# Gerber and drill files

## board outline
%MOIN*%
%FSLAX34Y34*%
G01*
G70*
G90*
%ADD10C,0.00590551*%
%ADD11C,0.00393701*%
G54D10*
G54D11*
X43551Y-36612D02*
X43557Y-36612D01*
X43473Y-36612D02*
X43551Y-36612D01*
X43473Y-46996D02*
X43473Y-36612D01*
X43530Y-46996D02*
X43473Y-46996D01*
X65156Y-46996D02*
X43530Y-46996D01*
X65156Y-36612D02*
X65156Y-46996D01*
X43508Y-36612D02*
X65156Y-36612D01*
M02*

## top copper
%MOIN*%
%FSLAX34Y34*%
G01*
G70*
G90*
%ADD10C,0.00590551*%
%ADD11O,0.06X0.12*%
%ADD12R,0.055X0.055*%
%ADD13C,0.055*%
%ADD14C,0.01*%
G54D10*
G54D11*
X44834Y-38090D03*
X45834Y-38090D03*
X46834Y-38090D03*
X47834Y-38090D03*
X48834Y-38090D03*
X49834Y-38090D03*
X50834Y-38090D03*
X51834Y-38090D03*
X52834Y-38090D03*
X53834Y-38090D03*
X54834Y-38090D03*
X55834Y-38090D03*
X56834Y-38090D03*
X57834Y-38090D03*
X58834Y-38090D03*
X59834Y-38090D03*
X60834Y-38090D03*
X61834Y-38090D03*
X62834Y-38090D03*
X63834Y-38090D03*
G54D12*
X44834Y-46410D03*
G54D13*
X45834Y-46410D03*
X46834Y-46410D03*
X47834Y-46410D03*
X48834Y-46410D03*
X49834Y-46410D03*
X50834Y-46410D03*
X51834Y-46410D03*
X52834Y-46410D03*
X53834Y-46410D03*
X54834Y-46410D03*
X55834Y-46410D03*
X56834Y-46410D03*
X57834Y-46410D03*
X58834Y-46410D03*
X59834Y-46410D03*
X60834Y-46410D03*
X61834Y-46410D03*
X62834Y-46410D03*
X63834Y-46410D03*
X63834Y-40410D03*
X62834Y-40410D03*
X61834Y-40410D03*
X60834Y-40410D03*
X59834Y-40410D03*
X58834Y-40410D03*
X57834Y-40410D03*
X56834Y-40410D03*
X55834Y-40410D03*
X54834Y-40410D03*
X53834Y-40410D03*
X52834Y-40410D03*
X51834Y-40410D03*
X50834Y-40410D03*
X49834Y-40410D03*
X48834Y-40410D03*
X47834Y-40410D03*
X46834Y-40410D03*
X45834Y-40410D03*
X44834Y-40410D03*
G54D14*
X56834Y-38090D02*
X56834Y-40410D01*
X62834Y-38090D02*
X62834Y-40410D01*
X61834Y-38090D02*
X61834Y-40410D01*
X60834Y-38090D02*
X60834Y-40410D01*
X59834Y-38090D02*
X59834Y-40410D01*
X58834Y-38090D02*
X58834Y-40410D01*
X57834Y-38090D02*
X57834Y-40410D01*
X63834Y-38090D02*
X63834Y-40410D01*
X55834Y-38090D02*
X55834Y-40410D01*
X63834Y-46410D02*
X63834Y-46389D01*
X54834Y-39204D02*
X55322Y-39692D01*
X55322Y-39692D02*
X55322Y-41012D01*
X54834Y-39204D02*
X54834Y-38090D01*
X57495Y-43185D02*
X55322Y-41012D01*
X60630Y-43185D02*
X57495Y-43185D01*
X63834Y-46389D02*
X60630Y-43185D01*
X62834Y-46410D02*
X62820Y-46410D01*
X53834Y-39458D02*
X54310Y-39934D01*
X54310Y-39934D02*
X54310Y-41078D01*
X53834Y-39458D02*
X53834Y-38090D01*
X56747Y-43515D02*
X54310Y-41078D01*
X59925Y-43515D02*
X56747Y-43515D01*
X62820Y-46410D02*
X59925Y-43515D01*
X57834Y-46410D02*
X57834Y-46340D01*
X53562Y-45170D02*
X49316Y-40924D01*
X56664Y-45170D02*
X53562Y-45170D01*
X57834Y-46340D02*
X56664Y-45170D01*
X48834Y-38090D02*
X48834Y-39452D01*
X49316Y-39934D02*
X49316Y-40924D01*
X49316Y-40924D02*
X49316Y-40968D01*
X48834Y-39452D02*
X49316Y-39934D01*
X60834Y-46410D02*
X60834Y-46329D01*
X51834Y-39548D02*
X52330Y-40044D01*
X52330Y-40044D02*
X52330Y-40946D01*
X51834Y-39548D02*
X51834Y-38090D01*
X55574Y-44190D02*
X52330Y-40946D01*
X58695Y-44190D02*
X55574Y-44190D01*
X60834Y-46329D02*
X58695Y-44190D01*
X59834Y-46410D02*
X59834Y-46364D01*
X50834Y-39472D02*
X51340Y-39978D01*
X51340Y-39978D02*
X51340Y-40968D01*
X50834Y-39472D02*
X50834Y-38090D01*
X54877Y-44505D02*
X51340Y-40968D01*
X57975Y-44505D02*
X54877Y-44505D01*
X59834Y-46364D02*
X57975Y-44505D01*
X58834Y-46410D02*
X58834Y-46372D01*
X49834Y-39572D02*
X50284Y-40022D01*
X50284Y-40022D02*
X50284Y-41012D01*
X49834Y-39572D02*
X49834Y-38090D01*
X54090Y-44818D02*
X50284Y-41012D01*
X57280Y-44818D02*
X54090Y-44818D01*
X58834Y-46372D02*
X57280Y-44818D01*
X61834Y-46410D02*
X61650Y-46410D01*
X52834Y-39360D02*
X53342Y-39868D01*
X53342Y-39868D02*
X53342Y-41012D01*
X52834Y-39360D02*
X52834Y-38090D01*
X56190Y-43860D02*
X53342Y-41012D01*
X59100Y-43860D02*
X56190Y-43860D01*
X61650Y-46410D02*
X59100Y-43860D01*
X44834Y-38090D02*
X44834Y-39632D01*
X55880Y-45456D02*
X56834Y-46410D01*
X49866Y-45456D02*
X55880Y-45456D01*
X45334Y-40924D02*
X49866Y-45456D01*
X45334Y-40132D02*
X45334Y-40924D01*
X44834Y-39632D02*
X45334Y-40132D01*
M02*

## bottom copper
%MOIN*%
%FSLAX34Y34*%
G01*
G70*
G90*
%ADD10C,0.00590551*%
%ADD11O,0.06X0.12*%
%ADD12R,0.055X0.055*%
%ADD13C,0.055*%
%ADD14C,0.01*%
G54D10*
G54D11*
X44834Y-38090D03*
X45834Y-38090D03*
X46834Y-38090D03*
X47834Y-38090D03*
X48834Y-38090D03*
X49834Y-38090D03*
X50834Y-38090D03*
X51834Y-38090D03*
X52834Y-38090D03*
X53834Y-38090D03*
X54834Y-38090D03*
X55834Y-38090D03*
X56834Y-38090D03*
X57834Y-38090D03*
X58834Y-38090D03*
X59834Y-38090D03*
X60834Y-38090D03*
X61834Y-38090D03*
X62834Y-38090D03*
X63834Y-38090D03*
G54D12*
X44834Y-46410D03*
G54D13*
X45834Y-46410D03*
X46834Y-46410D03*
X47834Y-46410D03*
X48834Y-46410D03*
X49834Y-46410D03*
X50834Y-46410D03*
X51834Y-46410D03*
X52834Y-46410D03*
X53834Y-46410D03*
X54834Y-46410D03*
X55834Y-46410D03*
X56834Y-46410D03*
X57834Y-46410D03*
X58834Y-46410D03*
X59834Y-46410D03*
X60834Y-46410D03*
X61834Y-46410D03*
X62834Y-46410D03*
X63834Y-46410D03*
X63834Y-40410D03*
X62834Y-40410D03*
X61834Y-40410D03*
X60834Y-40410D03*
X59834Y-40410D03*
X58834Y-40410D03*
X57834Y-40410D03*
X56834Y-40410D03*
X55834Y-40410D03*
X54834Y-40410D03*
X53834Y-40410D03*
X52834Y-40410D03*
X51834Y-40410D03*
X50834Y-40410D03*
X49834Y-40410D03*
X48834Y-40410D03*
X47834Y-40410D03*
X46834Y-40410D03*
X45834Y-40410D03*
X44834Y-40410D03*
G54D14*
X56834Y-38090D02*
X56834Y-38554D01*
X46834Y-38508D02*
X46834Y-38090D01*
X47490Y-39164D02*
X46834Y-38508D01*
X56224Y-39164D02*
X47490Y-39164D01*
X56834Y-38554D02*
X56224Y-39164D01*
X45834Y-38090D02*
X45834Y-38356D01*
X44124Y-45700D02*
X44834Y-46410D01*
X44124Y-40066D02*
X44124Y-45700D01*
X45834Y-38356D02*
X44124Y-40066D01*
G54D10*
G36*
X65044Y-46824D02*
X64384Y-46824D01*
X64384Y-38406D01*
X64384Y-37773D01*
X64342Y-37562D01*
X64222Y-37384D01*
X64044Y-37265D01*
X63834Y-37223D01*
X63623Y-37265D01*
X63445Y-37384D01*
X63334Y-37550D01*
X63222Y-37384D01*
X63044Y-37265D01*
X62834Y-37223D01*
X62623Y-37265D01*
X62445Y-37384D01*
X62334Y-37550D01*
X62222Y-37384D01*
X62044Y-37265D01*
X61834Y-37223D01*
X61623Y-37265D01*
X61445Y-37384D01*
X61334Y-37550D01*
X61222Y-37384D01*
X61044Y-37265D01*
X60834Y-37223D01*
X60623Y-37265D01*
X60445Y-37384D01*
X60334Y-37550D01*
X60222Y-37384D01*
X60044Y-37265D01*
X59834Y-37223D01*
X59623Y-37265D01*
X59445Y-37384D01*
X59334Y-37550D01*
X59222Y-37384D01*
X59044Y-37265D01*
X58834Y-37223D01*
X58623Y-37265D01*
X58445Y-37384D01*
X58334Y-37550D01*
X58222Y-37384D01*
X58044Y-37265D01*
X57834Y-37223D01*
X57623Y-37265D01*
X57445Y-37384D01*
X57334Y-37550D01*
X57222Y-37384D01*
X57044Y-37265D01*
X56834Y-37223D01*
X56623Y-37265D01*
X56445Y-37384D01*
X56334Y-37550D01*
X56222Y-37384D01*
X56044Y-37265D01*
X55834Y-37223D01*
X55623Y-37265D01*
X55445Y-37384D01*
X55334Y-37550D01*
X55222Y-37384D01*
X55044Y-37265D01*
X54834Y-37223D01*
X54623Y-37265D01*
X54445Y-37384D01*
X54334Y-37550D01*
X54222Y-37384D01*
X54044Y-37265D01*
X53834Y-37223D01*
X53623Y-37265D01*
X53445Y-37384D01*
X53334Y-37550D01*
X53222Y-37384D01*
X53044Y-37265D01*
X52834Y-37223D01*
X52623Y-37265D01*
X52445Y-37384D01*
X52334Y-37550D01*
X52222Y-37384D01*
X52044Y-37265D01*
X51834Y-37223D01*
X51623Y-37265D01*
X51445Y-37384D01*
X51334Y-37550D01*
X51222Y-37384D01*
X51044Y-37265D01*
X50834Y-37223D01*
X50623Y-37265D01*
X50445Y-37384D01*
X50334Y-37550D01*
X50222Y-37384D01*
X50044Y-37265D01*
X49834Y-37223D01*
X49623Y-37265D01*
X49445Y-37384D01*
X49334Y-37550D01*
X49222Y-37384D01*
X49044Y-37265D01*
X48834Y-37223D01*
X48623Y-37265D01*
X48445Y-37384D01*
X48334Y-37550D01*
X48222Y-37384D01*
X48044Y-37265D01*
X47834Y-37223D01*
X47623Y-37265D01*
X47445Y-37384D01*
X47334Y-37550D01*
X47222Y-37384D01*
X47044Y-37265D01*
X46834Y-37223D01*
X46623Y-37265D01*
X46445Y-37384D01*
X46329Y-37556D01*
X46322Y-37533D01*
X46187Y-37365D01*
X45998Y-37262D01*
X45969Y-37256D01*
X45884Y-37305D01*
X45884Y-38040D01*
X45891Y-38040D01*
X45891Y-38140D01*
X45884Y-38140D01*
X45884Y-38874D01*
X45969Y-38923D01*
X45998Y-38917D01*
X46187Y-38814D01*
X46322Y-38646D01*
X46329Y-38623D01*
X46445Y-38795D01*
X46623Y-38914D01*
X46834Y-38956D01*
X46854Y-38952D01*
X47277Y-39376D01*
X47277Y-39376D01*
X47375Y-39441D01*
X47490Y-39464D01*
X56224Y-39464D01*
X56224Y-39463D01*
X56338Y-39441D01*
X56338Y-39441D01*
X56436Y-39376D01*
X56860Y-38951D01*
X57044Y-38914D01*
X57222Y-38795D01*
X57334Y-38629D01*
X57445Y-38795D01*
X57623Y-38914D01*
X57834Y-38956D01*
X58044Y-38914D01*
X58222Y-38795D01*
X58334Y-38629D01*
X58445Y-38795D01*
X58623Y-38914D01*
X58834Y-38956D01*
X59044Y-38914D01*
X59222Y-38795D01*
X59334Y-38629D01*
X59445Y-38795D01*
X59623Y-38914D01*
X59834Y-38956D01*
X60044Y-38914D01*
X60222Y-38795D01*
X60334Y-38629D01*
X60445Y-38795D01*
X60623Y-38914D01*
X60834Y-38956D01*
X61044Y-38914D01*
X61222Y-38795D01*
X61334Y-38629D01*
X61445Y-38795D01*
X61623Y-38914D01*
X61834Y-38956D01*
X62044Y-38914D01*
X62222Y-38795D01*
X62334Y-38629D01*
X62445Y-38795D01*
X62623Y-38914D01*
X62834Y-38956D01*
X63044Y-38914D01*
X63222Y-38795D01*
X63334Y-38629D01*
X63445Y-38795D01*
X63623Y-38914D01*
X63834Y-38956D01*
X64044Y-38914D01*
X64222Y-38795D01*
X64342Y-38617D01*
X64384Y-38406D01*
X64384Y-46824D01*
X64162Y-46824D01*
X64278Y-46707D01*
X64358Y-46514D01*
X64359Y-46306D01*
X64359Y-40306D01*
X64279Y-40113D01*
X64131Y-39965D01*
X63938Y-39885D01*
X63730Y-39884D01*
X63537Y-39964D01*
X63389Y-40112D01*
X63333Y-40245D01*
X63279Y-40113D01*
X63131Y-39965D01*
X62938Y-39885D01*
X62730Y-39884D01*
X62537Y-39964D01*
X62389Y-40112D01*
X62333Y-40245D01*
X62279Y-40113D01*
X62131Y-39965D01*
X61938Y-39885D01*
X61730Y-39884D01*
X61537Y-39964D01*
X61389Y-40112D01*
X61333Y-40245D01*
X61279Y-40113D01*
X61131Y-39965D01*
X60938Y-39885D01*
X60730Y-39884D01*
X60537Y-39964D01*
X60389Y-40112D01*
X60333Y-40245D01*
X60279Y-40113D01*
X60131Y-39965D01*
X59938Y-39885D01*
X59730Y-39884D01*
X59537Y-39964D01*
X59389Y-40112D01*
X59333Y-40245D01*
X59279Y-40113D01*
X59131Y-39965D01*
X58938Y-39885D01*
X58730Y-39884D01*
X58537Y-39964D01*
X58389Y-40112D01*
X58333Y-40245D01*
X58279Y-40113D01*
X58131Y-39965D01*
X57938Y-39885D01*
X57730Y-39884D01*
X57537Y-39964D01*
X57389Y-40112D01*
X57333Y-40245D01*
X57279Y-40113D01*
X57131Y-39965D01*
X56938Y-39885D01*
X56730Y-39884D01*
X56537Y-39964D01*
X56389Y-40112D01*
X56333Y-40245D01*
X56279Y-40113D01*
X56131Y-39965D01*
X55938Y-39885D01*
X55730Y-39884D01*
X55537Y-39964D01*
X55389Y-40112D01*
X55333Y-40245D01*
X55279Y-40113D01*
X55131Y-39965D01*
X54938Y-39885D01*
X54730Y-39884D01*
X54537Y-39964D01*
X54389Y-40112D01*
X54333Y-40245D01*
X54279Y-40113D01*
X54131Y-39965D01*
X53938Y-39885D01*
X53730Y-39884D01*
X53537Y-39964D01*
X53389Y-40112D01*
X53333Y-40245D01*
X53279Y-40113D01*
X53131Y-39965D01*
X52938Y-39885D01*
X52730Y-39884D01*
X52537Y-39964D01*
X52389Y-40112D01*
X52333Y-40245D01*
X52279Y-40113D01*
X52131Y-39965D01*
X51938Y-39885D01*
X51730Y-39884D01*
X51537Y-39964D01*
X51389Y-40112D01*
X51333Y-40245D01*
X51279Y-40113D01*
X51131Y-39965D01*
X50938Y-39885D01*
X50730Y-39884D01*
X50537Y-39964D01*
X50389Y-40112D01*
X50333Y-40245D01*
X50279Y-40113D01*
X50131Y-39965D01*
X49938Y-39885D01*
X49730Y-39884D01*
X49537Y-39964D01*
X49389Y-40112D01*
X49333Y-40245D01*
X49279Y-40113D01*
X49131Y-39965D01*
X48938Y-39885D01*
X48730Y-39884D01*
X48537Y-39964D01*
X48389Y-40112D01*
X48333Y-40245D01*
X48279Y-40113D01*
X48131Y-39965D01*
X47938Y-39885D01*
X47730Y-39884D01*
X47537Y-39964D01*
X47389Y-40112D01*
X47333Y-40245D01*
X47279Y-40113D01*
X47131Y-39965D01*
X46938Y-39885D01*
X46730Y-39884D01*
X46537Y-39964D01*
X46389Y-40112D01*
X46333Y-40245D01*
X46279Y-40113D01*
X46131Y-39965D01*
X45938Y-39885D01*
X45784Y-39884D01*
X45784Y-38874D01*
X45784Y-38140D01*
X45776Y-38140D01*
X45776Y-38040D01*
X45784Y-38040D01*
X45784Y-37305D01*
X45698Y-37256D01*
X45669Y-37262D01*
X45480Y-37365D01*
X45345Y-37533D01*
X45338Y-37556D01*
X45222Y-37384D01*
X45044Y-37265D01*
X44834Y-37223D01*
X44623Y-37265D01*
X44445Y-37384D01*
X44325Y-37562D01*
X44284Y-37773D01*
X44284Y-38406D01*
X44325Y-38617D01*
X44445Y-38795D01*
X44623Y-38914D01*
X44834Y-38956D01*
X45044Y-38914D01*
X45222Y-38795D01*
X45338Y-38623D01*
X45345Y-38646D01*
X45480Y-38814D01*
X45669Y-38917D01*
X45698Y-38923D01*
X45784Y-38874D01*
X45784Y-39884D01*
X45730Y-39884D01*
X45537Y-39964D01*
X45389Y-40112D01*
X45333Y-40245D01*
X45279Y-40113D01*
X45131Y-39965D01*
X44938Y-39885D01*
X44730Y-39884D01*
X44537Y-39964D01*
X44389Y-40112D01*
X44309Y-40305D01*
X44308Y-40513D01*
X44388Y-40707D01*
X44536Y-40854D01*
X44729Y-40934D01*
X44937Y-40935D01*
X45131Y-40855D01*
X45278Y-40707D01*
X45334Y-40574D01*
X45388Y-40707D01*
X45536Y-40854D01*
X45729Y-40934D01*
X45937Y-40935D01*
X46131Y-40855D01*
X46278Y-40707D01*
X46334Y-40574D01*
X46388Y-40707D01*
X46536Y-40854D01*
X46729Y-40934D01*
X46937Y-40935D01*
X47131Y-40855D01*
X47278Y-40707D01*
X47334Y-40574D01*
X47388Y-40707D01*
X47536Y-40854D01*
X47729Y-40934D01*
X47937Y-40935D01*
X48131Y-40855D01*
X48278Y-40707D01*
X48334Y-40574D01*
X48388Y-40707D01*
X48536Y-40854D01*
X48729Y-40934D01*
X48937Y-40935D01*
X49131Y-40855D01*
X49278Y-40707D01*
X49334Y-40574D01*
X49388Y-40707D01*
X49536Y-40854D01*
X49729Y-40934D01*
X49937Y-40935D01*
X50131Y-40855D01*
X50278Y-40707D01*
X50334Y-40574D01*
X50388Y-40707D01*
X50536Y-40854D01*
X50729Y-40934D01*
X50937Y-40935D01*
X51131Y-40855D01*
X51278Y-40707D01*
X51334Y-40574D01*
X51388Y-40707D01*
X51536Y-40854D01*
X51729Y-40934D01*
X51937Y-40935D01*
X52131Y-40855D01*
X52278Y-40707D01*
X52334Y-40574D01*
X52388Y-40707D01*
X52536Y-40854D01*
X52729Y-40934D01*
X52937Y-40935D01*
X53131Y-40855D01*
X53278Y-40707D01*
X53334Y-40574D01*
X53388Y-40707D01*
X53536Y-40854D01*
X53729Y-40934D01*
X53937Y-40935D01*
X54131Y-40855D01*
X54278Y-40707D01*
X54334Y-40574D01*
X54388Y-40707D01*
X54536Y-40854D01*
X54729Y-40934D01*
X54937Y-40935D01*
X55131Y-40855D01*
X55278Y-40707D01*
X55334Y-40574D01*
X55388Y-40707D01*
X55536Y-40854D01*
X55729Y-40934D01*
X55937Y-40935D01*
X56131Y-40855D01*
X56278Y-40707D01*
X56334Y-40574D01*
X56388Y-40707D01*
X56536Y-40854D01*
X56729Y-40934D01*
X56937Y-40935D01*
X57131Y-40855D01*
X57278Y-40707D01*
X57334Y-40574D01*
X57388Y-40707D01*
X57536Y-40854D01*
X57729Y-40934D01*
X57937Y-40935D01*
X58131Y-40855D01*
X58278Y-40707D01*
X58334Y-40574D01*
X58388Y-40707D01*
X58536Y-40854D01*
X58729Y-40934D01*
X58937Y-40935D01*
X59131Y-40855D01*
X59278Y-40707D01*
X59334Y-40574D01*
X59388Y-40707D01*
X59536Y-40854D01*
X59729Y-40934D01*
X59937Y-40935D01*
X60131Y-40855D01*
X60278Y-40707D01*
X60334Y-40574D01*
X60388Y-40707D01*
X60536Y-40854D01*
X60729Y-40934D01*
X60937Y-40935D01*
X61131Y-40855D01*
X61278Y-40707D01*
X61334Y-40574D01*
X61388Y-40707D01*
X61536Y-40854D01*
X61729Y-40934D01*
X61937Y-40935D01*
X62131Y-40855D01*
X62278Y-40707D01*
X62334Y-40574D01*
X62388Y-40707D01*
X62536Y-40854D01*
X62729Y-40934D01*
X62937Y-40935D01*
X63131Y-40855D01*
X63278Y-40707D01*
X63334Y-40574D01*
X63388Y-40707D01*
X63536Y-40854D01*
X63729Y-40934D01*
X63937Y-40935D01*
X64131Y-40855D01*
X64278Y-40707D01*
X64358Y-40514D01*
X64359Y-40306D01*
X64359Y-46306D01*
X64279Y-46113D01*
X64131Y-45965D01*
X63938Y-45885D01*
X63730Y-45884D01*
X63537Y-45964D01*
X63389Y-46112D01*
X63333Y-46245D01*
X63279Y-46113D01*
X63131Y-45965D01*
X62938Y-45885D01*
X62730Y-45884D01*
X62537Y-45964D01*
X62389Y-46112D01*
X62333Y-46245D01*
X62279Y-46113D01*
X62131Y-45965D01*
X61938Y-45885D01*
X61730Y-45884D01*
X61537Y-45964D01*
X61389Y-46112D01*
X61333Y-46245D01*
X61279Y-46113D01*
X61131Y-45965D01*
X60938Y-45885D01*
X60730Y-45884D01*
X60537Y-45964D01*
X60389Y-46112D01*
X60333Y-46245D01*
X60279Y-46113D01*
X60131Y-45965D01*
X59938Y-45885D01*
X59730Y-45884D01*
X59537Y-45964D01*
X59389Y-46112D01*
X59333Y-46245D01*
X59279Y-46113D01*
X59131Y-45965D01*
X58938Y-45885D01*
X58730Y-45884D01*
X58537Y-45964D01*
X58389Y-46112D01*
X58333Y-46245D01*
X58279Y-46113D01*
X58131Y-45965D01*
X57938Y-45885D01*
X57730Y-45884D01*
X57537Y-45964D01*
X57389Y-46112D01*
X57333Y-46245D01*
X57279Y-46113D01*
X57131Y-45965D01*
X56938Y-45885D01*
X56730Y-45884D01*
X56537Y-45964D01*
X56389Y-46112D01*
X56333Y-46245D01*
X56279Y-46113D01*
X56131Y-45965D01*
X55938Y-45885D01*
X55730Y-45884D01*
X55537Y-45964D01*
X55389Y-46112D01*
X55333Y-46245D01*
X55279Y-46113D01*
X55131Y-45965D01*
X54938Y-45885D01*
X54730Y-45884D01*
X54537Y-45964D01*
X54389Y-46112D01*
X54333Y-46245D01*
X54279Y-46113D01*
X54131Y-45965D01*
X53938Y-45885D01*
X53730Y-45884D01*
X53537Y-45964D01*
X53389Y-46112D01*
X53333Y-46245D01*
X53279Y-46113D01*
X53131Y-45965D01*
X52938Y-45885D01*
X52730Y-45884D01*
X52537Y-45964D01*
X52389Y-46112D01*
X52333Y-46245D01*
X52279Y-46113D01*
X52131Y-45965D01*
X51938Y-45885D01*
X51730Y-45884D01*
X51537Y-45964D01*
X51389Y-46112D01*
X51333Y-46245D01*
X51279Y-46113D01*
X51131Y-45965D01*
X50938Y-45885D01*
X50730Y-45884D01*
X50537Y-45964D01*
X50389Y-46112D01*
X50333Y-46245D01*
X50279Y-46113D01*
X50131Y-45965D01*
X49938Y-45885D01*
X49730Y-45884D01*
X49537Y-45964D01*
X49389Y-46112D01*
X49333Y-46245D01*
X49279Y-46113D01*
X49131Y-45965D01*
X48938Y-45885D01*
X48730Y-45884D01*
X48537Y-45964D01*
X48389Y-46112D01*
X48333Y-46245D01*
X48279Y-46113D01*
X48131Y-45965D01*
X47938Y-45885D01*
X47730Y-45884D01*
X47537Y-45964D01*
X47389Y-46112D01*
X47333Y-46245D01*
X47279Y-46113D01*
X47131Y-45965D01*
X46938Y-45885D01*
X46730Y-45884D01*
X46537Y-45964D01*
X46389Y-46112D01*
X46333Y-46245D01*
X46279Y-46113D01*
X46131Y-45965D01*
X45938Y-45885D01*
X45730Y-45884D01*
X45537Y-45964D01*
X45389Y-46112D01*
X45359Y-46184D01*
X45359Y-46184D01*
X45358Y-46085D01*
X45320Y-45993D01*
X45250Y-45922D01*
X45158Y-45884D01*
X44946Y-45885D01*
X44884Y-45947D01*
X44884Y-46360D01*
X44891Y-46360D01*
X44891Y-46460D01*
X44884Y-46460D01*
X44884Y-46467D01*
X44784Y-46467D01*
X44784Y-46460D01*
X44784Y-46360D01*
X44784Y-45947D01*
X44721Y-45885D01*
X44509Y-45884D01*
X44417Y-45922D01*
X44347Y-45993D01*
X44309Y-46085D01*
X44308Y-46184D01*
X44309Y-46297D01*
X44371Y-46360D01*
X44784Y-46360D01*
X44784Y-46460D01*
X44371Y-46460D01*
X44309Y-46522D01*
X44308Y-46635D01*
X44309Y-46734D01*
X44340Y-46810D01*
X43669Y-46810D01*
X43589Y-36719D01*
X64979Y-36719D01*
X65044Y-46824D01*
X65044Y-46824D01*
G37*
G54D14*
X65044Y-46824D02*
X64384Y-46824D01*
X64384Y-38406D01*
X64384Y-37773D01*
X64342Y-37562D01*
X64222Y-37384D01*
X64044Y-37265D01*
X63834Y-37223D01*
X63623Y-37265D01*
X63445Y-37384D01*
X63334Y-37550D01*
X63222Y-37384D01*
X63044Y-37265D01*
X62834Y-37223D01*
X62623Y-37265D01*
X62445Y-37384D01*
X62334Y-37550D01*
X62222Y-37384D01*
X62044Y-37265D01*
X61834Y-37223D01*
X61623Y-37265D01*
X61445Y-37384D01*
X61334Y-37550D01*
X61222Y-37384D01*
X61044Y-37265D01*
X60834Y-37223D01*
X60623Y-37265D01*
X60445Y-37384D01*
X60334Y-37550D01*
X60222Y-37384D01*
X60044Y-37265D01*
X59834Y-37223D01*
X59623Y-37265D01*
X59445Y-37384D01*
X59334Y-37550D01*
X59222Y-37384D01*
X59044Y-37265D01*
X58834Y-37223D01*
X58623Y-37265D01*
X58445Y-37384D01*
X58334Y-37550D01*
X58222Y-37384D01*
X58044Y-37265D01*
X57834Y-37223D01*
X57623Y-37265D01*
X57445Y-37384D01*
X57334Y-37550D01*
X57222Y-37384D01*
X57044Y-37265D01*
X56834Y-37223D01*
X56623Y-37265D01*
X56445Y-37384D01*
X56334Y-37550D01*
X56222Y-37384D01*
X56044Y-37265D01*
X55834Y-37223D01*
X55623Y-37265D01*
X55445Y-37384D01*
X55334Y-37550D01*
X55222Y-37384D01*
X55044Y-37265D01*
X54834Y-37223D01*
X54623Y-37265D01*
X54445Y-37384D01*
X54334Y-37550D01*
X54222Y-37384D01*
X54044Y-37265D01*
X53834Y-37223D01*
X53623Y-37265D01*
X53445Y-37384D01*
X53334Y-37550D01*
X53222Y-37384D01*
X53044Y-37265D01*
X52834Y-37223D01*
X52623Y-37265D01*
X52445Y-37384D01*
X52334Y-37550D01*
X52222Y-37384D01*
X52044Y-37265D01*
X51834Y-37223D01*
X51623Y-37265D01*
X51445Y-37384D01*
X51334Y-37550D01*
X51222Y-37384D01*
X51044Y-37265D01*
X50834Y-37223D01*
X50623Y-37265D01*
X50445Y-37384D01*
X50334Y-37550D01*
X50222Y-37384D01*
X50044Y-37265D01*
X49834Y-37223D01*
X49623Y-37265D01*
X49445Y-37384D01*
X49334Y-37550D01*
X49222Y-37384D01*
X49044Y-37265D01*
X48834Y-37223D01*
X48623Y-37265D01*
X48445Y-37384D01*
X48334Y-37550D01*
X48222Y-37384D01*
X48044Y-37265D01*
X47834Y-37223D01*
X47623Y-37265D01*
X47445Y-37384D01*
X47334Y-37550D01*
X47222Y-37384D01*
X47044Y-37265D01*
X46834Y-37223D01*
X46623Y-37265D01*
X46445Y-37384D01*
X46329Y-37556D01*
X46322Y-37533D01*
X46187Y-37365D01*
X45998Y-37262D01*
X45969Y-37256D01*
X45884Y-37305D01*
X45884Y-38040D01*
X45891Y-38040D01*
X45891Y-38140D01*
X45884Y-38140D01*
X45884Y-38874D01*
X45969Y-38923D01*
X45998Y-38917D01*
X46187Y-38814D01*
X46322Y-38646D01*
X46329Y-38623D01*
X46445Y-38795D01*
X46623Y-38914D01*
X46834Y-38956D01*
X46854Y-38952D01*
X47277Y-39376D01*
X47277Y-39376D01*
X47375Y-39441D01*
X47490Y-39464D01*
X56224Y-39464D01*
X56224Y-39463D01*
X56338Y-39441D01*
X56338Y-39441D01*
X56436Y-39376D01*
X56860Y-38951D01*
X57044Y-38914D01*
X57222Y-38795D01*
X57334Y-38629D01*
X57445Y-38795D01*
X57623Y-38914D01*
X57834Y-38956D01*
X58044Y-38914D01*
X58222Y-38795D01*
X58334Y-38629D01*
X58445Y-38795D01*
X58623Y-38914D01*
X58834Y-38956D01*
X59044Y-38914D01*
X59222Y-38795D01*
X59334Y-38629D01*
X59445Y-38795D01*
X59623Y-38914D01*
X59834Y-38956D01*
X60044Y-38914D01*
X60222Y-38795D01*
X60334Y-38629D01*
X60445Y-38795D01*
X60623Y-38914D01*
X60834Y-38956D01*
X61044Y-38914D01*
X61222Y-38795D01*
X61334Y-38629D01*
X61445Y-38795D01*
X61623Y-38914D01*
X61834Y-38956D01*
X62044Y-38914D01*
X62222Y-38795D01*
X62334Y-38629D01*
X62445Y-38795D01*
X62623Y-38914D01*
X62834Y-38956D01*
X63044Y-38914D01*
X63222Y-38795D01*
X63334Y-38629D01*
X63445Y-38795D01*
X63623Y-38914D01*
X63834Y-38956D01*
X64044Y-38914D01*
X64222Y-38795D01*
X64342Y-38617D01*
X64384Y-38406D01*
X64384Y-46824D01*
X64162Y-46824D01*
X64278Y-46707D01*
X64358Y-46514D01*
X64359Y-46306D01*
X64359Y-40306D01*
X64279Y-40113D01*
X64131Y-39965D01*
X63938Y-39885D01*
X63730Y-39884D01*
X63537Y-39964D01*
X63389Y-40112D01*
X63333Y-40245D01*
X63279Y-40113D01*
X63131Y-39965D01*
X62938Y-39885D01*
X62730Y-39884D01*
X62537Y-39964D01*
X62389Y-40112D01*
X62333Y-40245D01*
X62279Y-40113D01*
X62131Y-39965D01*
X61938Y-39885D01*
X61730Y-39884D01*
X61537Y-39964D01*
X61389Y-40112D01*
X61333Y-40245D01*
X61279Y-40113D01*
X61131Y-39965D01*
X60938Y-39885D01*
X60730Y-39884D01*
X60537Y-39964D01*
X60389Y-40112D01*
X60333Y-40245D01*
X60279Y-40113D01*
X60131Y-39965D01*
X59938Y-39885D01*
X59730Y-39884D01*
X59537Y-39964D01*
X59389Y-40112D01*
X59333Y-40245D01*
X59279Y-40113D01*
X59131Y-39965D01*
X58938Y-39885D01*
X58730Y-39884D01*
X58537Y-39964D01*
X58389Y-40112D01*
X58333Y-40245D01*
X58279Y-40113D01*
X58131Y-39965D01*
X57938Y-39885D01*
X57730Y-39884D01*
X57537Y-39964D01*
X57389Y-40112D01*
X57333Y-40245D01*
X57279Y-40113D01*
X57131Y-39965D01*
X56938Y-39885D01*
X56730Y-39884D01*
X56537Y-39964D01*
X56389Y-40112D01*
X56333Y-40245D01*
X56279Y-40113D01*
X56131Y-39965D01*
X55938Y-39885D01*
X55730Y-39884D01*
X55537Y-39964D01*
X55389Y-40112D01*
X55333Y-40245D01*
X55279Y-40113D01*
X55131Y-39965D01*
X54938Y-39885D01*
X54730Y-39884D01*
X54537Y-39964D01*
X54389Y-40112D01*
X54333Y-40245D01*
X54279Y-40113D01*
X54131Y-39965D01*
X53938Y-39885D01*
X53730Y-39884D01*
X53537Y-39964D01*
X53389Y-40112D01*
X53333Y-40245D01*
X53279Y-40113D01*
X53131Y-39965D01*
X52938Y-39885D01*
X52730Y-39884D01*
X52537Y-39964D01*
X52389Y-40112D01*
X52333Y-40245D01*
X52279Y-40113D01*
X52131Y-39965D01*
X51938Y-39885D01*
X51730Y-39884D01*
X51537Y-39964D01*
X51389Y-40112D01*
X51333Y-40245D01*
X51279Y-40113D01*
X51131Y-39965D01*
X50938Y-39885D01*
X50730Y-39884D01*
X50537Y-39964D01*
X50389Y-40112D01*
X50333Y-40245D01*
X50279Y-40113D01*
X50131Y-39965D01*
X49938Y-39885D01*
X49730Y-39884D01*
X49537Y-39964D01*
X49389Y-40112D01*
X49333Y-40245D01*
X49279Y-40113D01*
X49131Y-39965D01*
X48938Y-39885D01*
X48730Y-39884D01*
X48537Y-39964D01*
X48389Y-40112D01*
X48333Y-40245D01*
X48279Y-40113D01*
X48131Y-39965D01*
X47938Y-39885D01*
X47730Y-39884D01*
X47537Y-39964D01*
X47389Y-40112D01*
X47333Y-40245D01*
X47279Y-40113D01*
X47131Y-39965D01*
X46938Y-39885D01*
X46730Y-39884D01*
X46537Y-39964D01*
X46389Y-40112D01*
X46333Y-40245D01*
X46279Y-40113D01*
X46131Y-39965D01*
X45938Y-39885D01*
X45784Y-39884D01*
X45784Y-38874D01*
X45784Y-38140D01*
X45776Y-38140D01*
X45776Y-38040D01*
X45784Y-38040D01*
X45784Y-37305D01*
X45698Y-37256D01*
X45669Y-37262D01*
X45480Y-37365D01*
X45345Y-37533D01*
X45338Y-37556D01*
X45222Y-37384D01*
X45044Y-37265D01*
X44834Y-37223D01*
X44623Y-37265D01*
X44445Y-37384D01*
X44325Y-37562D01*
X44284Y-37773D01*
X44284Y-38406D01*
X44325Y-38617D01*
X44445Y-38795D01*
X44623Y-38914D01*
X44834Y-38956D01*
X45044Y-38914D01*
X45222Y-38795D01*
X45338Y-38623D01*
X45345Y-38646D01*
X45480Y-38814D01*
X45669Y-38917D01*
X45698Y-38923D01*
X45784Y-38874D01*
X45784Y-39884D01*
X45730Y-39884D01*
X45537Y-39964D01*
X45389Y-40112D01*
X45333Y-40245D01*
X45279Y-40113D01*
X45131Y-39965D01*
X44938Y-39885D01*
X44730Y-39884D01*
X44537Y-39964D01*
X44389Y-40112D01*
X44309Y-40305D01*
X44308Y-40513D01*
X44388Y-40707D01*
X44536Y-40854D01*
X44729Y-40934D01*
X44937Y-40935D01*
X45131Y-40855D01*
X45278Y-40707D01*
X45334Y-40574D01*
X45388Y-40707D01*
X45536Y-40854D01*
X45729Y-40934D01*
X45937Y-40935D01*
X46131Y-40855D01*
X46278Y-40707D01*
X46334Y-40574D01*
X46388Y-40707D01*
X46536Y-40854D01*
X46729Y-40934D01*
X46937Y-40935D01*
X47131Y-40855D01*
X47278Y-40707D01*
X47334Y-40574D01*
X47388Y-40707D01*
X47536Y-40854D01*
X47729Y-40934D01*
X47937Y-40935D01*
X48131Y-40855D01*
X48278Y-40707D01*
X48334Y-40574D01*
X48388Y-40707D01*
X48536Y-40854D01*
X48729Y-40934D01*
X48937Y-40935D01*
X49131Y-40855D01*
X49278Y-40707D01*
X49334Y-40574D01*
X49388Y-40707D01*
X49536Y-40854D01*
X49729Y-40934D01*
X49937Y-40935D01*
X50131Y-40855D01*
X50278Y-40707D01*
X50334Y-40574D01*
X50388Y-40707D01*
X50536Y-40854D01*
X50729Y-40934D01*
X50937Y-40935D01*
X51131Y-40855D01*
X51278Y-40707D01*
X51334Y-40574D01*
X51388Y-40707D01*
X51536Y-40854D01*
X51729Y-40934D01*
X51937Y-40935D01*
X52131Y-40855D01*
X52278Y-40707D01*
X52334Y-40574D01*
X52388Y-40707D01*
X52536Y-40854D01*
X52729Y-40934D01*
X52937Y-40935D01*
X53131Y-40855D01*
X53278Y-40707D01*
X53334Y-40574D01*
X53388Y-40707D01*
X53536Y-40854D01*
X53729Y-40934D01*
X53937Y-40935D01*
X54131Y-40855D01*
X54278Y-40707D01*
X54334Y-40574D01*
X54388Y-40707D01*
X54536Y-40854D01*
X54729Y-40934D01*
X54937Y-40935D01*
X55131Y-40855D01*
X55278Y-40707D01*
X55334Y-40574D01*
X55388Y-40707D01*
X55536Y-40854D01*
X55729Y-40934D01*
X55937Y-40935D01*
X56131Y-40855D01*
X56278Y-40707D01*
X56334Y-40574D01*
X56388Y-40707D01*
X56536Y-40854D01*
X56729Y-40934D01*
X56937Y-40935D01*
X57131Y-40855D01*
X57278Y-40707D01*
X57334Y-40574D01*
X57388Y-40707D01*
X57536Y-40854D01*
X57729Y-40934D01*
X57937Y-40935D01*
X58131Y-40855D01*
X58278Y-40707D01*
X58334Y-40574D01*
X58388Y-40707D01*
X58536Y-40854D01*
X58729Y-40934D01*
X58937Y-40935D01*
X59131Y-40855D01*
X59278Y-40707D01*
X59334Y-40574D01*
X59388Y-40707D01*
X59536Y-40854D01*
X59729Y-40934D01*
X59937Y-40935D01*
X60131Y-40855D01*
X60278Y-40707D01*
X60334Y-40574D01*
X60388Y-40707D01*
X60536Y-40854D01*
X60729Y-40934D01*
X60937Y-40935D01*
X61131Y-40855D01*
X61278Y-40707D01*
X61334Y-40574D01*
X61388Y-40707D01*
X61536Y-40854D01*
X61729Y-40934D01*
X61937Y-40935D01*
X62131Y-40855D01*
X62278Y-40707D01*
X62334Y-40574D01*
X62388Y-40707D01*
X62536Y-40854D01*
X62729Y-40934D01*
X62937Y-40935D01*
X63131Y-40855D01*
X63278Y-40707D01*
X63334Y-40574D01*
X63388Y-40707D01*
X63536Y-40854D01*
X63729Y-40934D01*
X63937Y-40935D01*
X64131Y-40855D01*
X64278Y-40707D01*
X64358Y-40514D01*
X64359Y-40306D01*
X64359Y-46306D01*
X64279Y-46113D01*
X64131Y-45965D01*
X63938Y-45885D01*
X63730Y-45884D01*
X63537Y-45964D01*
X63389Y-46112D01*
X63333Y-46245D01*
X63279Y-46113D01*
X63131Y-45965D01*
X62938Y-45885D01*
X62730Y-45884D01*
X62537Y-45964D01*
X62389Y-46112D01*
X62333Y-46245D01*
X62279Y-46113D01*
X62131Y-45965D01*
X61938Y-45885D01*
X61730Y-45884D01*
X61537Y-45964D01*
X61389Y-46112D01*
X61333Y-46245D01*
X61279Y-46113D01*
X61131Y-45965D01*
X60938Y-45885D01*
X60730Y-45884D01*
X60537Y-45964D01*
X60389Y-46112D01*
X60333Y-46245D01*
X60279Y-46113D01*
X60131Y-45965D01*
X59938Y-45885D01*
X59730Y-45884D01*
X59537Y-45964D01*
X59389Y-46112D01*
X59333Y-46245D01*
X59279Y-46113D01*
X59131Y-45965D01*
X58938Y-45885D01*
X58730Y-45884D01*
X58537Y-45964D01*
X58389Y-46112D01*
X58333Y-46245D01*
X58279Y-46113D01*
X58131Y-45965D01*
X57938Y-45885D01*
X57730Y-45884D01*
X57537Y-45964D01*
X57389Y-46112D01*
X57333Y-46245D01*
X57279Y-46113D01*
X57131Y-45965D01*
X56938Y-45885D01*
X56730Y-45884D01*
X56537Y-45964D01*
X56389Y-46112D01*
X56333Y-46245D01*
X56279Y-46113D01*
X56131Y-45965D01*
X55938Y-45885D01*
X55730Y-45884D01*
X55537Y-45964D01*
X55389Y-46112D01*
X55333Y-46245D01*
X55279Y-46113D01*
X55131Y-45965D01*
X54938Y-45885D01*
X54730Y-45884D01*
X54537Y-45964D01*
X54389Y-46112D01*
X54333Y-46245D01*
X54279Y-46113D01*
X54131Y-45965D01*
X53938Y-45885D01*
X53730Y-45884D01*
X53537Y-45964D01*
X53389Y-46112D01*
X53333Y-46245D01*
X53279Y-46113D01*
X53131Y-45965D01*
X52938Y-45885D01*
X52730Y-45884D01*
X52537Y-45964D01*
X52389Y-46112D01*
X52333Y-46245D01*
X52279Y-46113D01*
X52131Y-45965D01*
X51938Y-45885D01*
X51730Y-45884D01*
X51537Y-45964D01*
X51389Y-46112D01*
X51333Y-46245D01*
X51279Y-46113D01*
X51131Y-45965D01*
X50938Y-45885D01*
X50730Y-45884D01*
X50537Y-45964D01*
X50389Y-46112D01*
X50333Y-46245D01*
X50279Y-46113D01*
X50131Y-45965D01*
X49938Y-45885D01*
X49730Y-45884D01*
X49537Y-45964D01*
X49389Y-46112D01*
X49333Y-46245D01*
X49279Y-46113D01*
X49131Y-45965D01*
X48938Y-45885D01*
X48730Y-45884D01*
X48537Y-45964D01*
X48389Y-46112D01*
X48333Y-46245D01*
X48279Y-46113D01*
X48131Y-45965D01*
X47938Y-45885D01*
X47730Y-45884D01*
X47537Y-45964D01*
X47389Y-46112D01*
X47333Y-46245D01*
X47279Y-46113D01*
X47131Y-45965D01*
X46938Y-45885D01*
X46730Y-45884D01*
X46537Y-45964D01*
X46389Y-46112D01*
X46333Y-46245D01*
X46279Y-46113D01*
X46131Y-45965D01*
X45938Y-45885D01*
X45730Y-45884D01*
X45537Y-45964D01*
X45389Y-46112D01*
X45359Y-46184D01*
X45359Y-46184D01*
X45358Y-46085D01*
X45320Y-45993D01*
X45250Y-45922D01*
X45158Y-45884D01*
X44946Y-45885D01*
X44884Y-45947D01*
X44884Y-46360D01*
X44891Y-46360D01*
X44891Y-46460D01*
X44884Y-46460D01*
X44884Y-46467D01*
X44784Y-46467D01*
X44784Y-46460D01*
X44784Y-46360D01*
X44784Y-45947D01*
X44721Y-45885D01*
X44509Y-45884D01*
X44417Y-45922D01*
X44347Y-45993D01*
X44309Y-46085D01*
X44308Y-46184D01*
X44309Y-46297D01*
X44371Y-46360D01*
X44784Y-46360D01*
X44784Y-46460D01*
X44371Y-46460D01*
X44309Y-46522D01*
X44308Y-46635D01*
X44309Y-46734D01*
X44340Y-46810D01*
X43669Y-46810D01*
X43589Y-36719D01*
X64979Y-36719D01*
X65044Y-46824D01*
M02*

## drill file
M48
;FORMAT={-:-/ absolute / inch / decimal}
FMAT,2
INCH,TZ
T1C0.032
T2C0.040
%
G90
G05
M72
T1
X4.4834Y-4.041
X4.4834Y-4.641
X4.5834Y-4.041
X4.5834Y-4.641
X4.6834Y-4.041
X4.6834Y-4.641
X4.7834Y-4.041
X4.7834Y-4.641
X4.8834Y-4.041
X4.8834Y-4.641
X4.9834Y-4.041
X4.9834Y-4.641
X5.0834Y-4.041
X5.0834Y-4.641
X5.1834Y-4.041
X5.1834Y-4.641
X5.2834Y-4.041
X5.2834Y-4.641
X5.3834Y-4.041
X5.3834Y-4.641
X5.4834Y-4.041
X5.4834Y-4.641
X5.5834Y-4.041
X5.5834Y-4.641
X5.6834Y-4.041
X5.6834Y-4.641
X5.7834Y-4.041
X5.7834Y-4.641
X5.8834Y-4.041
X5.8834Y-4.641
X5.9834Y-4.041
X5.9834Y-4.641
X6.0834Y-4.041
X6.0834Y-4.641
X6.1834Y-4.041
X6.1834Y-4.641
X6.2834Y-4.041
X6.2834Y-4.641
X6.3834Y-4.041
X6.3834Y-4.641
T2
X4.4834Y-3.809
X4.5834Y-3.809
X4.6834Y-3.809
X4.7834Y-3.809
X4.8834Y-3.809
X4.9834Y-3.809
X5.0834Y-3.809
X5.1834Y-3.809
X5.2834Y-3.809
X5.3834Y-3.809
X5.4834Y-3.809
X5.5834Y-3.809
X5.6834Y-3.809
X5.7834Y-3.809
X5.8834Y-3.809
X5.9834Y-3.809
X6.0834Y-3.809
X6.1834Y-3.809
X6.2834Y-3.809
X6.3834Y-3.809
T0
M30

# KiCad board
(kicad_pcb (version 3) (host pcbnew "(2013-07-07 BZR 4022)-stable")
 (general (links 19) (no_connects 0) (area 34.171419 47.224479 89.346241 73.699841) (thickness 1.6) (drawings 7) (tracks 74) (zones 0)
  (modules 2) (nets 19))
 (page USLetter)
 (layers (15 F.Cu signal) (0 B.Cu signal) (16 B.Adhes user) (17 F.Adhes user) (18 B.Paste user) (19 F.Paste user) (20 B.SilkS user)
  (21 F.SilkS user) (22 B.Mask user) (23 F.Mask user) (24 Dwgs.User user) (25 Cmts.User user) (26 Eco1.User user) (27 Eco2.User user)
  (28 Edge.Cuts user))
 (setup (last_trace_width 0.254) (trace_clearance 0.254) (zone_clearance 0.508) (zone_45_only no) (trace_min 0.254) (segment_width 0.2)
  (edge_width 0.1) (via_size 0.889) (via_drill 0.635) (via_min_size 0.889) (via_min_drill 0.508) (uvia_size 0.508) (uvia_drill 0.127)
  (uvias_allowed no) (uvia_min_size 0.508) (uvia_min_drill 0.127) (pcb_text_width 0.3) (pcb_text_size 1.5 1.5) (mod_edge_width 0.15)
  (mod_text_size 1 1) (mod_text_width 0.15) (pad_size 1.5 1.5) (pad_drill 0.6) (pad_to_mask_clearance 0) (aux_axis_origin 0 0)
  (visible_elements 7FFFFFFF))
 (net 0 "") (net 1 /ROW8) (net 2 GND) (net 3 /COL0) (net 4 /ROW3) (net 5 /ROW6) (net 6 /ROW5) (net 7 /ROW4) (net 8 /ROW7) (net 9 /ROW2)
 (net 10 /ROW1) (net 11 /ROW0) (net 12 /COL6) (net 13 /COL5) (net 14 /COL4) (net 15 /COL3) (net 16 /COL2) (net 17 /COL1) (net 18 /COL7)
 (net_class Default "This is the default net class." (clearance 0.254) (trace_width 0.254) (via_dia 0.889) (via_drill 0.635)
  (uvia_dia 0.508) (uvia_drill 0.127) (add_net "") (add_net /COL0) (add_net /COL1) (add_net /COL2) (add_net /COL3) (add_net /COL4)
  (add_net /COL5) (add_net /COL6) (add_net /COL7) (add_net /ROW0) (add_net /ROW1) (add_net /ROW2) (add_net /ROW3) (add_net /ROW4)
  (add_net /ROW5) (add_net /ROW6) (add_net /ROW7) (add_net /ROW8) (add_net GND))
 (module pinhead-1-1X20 (layer F.Cu) (at 138.00836 96.7486)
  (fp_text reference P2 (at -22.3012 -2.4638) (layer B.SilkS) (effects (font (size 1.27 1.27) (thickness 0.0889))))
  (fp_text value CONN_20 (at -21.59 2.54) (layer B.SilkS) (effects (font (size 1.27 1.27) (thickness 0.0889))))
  (pad 1 thru_hole oval (at -24.13 0) (size 1.524 3.048) (drill 1.016) (layers *.Cu F.Paste F.SilkS F.Mask) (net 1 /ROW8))
  (pad 2 thru_hole oval (at -21.59 0) (size 1.524 3.048) (drill 1.016) (layers *.Cu F.Paste F.SilkS F.Mask) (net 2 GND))
  (pad 3 thru_hole oval (at -19.05 0) (size 1.524 3.048) (drill 1.016) (layers *.Cu F.Paste F.SilkS F.Mask) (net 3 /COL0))
  (pad 4 thru_hole oval (at -16.51 0) (size 1.524 3.048) (drill 1.016) (layers *.Cu F.Paste F.SilkS F.Mask))
  (pad 5 thru_hole oval (at -13.97 0) (size 1.524 3.048) (drill 1.016) (layers *.Cu F.Paste F.SilkS F.Mask) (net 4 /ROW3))
  (pad 6 thru_hole oval (at -11.43 0) (size 1.524 3.048) (drill 1.016) (layers *.Cu F.Paste F.SilkS F.Mask) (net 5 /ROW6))
  (pad 7 thru_hole oval (at -8.89 0) (size 1.524 3.048) (drill 1.016) (layers *.Cu F.Paste F.SilkS F.Mask) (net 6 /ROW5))
  (pad 8 thru_hole oval (at -6.35 0) (size 1.524 3.048) (drill 1.016) (layers *.Cu F.Paste F.SilkS F.Mask) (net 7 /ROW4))
  (pad 9 thru_hole oval (at -3.81 0) (size 1.524 3.048) (drill 1.016) (layers *.Cu F.Paste F.SilkS F.Mask) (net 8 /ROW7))
  (pad 10 thru_hole oval (at -1.27 0) (size 1.524 3.048) (drill 1.016) (layers *.Cu F.Paste F.SilkS F.Mask) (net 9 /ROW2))
  (pad 11 thru_hole oval (at 1.27 0) (size 1.524 3.048) (drill 1.016) (layers *.Cu F.Paste F.SilkS F.Mask) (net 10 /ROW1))
  (pad 12 thru_hole oval (at 3.81 0) (size 1.524 3.048) (drill 1.016) (layers *.Cu F.Paste F.SilkS F.Mask) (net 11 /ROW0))
  (pad 13 thru_hole oval (at 6.35 0) (size 1.524 3.048) (drill 1.016) (layers *.Cu F.Paste F.SilkS F.Mask) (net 3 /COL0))
  (pad 14 thru_hole oval (at 8.89 0) (size 1.524 3.048) (drill 1.016) (layers *.Cu F.Paste F.SilkS F.Mask) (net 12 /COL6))
  (pad 15 thru_hole oval (at 11.43 0) (size 1.524 3.048) (drill 1.016) (layers *.Cu F.Paste F.SilkS F.Mask) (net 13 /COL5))
  (pad 16 thru_hole oval (at 13.97 0) (size 1.524 3.048) (drill 1.016) (layers *.Cu F.Paste F.SilkS F.Mask) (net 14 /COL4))
  (pad 17 thru_hole oval (at 16.51 0) (size 1.524 3.048) (drill 1.016) (layers *.Cu F.Paste F.SilkS F.Mask) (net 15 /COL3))
  (pad 18 thru_hole oval (at 19.05 0) (size 1.524 3.048) (drill 1.016) (layers *.Cu F.Paste F.SilkS F.Mask) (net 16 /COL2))
  (pad 19 thru_hole oval (at 21.59 0) (size 1.524 3.048) (drill 1.016) (layers *.Cu F.Paste F.SilkS F.Mask) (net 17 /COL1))
  (pad 20 thru_hole oval (at 24.13 0) (size 1.524 3.048) (drill 1.016) (layers *.Cu F.Paste F.SilkS F.Mask) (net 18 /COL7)))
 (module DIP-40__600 (layer F.Cu) (at 138.00836 110.2614)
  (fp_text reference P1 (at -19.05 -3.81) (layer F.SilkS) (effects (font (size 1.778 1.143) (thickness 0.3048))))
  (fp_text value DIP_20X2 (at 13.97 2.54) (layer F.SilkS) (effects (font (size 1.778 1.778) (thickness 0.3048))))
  (pad 1 thru_hole rect (at -24.13 7.62) (size 1.397 1.397) (drill 0.8128) (layers *.Cu *.Mask F.SilkS) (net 2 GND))
  (pad 2 thru_hole circle (at -21.59 7.62) (size 1.397 1.397) (drill 0.8128) (layers *.Cu *.Mask F.SilkS))
  (pad 3 thru_hole circle (at -19.05 7.62) (size 1.397 1.397) (drill 0.8128) (layers *.Cu *.Mask F.SilkS))
  (pad 4 thru_hole circle (at -16.51 7.62) (size 1.397 1.397) (drill 0.8128) (layers *.Cu *.Mask F.SilkS))
  (pad 5 thru_hole circle (at -13.97 7.62) (size 1.397 1.397) (drill 0.8128) (layers *.Cu *.Mask F.SilkS))
  (pad 6 thru_hole circle (at -11.43 7.62) (size 1.397 1.397) (drill 0.8128) (layers *.Cu *.Mask F.SilkS))
  (pad 7 thru_hole circle (at -8.89 7.62) (size 1.397 1.397) (drill 0.8128) (layers *.Cu *.Mask F.SilkS))
  (pad 8 thru_hole circle (at -6.35 7.62) (size 1.397 1.397) (drill 0.8128) (layers *.Cu *.Mask F.SilkS))
  (pad 9 thru_hole circle (at -3.81 7.62) (size 1.397 1.397) (drill 0.8128) (layers *.Cu *.Mask F.SilkS))
  (pad 10 thru_hole circle (at -1.27 7.62) (size 1.397 1.397) (drill 0.8128) (layers *.Cu *.Mask F.SilkS))
  (pad 11 thru_hole circle (at 1.27 7.62) (size 1.397 1.397) (drill 0.8128) (layers *.Cu *.Mask F.SilkS))
  (pad 12 thru_hole circle (at 3.81 7.62) (size 1.397 1.397) (drill 0.8128) (layers *.Cu *.Mask F.SilkS))
  (pad 13 thru_hole circle (at 6.35 7.62) (size 1.397 1.397) (drill 0.8128) (layers *.Cu *.Mask F.SilkS) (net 1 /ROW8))
  (pad 14 thru_hole circle (at 8.89 7.62) (size 1.397 1.397) (drill 0.8128) (layers *.Cu *.Mask F.SilkS) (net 4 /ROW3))
  (pad 15 thru_hole circle (at 11.43 7.62) (size 1.397 1.397) (drill 0.8128) (layers *.Cu *.Mask F.SilkS) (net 5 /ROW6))
  (pad 16 thru_hole circle (at 13.97 7.62) (size 1.397 1.397) (drill 0.8128) (layers *.Cu *.Mask F.SilkS) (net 6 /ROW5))
  (pad 17 thru_hole circle (at 16.51 7.62) (size 1.397 1.397) (drill 0.8128) (layers *.Cu *.Mask F.SilkS) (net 7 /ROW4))
  (pad 18 thru_hole circle (at 19.05 7.62) (size 1.397 1.397) (drill 0.8128) (layers *.Cu *.Mask F.SilkS) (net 8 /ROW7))
  (pad 19 thru_hole circle (at 21.59 7.62) (size 1.397 1.397) (drill 0.8128) (layers *.Cu *.Mask F.SilkS) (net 9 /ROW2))
  (pad 20 thru_hole circle (at 24.13 7.62) (size 1.397 1.397) (drill 0.8128) (layers *.Cu *.Mask F.SilkS) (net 10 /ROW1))
  (pad 21 thru_hole circle (at 24.13 -7.62) (size 1.397 1.397) (drill 0.8128) (layers *.Cu *.Mask F.SilkS) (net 18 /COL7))
  (pad 22 thru_hole circle (at 21.59 -7.62) (size 1.397 1.397) (drill 0.8128) (layers *.Cu *.Mask F.SilkS) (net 17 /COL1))
  (pad 23 thru_hole circle (at 19.05 -7.62) (size 1.397 1.397) (drill 0.8128) (layers *.Cu *.Mask F.SilkS) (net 16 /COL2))
  (pad 24 thru_hole circle (at 16.51 -7.62) (size 1.397 1.397) (drill 0.8128) (layers *.Cu *.Mask F.SilkS) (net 15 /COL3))
  (pad 25 thru_hole circle (at 13.97 -7.62) (size 1.397 1.397) (drill 0.8128) (layers *.Cu *.Mask F.SilkS) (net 14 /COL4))
  (pad 26 thru_hole circle (at 11.43 -7.62) (size 1.397 1.397) (drill 0.8128) (layers *.Cu *.Mask F.SilkS) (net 13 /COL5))
  (pad 27 thru_hole circle (at 8.89 -7.62) (size 1.397 1.397) (drill 0.8128) (layers *.Cu *.Mask F.SilkS) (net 12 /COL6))
  (pad 28 thru_hole circle (at 6.35 -7.62) (size 1.397 1.397) (drill 0.8128) (layers *.Cu *.Mask F.SilkS) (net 3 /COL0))
  (pad 29 thru_hole circle (at 3.81 -7.62) (size 1.397 1.397) (drill 0.8128) (layers *.Cu *.Mask F.SilkS) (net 11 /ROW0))
  (pad 30 thru_hole circle (at 1.27 -7.62) (size 1.397 1.397) (drill 0.8128) (layers *.Cu *.Mask F.SilkS))
  (pad 31 thru_hole circle (at -1.27 -7.62) (size 1.397 1.397) (drill 0.8128) (layers *.Cu *.Mask F.SilkS))
  (pad 32 thru_hole circle (at -3.81 -7.62) (size 1.397 1.397) (drill 0.8128) (layers *.Cu *.Mask F.SilkS))
  (pad 33 thru_hole circle (at -6.35 -7.62) (size 1.397 1.397) (drill 0.8128) (layers *.Cu *.Mask F.SilkS))
  (pad 34 thru_hole circle (at -8.89 -7.62) (size 1.397 1.397) (drill 0.8128) (layers *.Cu *.Mask F.SilkS))
  (pad 35 thru_hole circle (at -11.43 -7.62) (size 1.397 1.397) (drill 0.8128) (layers *.Cu *.Mask F.SilkS))
  (pad 36 thru_hole circle (at -13.97 -7.62) (size 1.397 1.397) (drill 0.8128) (layers *.Cu *.Mask F.SilkS))
  (pad 37 thru_hole circle (at -16.51 -7.62) (size 1.397 1.397) (drill 0.8128) (layers *.Cu *.Mask F.SilkS))
  (pad 38 thru_hole circle (at -19.05 -7.62) (size 1.397 1.397) (drill 0.8128) (layers *.Cu *.Mask F.SilkS))
  (pad 39 thru_hole circle (at -21.59 -7.62) (size 1.397 1.397) (drill 0.8128) (layers *.Cu *.Mask F.SilkS))
  (pad 40 thru_hole circle (at -24.13 -7.62) (size 1.397 1.397) (drill 0.8128) (layers *.Cu *.Mask F.SilkS)))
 (gr_line (start 110.61954 92.99448) (end 110.63478 92.99448) (angle 90) (layer Edge.Cuts) (width 0.1))
 (gr_line (start 110.42142 92.99448) (end 110.61954 92.99448) (angle 90) (layer Edge.Cuts) (width 0.1))
 (gr_line (start 110.42142 119.36984) (end 110.42142 92.99448) (angle 90) (layer Edge.Cuts) (width 0.1))
 (gr_line (start 110.5662 119.36984) (end 110.42142 119.36984) (angle 90) (layer Edge.Cuts) (width 0.1))
 (gr_line (start 165.49624 119.36984) (end 110.5662 119.36984) (angle 90) (layer Edge.Cuts) (width 0.1))
 (gr_line (start 165.49624 92.99448) (end 165.49624 119.36984) (angle 90) (layer Edge.Cuts) (width 0.1))
 (gr_line (start 110.51032 92.99448) (end 165.49624 92.99448) (angle 90) (layer Edge.Cuts) (width 0.1))
 (segment (start 144.35836 96.7486) (end 144.35836 97.92716) (width 0.254) (layer B.Cu) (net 3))
 (segment (start 118.95836 97.81032) (end 118.95836 96.7486) (width 0.254) (layer B.Cu) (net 3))
 (segment (start 120.6246 99.47656) (end 118.95836 97.81032) (width 0.254) (layer B.Cu) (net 3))
 (segment (start 142.80896 99.47656) (end 120.6246 99.47656) (width 0.254) (layer B.Cu) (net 3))
 (segment (start 144.35836 97.92716) (end 142.80896 99.47656) (width 0.254) (layer B.Cu) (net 3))
 (segment (start 144.35836 96.7486) (end 144.35836 102.6414) (width 0.254) (layer F.Cu) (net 3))
 (segment (start 159.59836 96.7486) (end 159.59836 102.6414) (width 0.254) (layer F.Cu) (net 17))
 (segment (start 157.05836 96.7486) (end 157.05836 102.6414) (width 0.254) (layer F.Cu) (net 16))
 (segment (start 154.51836 96.7486) (end 154.51836 102.6414) (width 0.254) (layer F.Cu) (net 15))
 (segment (start 151.97836 96.7486) (end 151.97836 102.6414) (width 0.254) (layer F.Cu) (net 14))
 (segment (start 149.43836 96.7486) (end 149.43836 102.6414) (width 0.254) (layer F.Cu) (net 13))
 (segment (start 146.89836 96.7486) (end 146.89836 102.6414) (width 0.254) (layer F.Cu) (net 12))
 (segment (start 162.13836 96.7486) (end 162.13836 102.6414) (width 0.254) (layer F.Cu) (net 18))
 (segment (start 141.81836 96.7486) (end 141.81836 102.6414) (width 0.254) (layer F.Cu) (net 11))
 (segment (start 162.13836 117.8814) (end 162.13836 117.82806) (width 0.254) (layer F.Cu) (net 10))
 (segment (start 139.27836 99.57816) (end 140.51788 100.81768) (width 0.254) (layer F.Cu) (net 10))
 (segment (start 140.51788 100.81768) (end 140.51788 104.17048) (width 0.254) (layer F.Cu) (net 10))
 (segment (start 139.27836 99.57816) (end 139.27836 96.7486) (width 0.254) (layer F.Cu) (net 10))
 (segment (start 146.0373 109.6899) (end 140.51788 104.17048) (width 0.254) (layer F.Cu) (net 10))
 (segment (start 154.0002 109.6899) (end 146.0373 109.6899) (width 0.254) (layer F.Cu) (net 10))
 (segment (start 162.13836 117.82806) (end 154.0002 109.6899) (width 0.254) (layer F.Cu) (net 10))
 (segment (start 159.59836 117.8814) (end 159.5628 117.8814) (width 0.254) (layer F.Cu) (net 9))
 (segment (start 136.73836 100.22332) (end 137.9474 101.43236) (width 0.254) (layer F.Cu) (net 9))
 (segment (start 137.9474 101.43236) (end 137.9474 104.33812) (width 0.254) (layer F.Cu) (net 9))
 (segment (start 136.73836 100.22332) (end 136.73836 96.7486) (width 0.254) (layer F.Cu) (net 9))
 (segment (start 144.13738 110.5281) (end 137.9474 104.33812) (width 0.254) (layer F.Cu) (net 9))
 (segment (start 152.2095 110.5281) (end 144.13738 110.5281) (width 0.254) (layer F.Cu) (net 9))
 (segment (start 159.5628 117.8814) (end 152.2095 110.5281) (width 0.254) (layer F.Cu) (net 9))
 (segment (start 146.89836 117.8814) (end 146.89836 117.7036) (width 0.254) (layer F.Cu) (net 4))
 (segment (start 136.04748 114.7318) (end 125.26264 103.94696) (width 0.254) (layer F.Cu) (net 4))
 (segment (start 143.92656 114.7318) (end 136.04748 114.7318) (width 0.254) (layer F.Cu) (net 4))
 (segment (start 146.89836 117.7036) (end 143.92656 114.7318) (width 0.254) (layer F.Cu) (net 4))
 (segment (start 124.03836 96.7486) (end 124.03836 100.20808) (width 0.254) (layer F.Cu) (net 4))
 (segment (start 125.26264 101.43236) (end 125.26264 103.94696) (width 0.254) (layer F.Cu) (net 4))
 (segment (start 125.26264 103.94696) (end 125.26264 104.05872) (width 0.254) (layer F.Cu) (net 4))
 (segment (start 124.03836 100.20808) (end 125.26264 101.43236) (width 0.254) (layer F.Cu) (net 4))
 (segment (start 154.51836 117.8814) (end 154.51836 117.67566) (width 0.254) (layer F.Cu) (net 7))
 (segment (start 131.65836 100.45192) (end 132.9182 101.71176) (width 0.254) (layer F.Cu) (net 7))
 (segment (start 132.9182 101.71176) (end 132.9182 104.00284) (width 0.254) (layer F.Cu) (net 7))
 (segment (start 131.65836 100.45192) (end 131.65836 96.7486) (width 0.254) (layer F.Cu) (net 7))
 (segment (start 141.15796 112.2426) (end 132.9182 104.00284) (width 0.254) (layer F.Cu) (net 7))
 (segment (start 149.0853 112.2426) (end 141.15796 112.2426) (width 0.254) (layer F.Cu) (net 7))
 (segment (start 154.51836 117.67566) (end 149.0853 112.2426) (width 0.254) (layer F.Cu) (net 7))
 (segment (start 151.97836 117.8814) (end 151.97836 117.76456) (width 0.254) (layer F.Cu) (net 6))
 (segment (start 129.11836 100.25888) (end 130.4036 101.54412) (width 0.254) (layer F.Cu) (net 6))
 (segment (start 130.4036 101.54412) (end 130.4036 104.05872) (width 0.254) (layer F.Cu) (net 6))
 (segment (start 129.11836 100.25888) (end 129.11836 96.7486) (width 0.254) (layer F.Cu) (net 6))
 (segment (start 139.38758 113.0427) (end 130.4036 104.05872) (width 0.254) (layer F.Cu) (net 6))
 (segment (start 147.2565 113.0427) (end 139.38758 113.0427) (width 0.254) (layer F.Cu) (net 6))
 (segment (start 151.97836 117.76456) (end 147.2565 113.0427) (width 0.254) (layer F.Cu) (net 6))
 (segment (start 149.43836 117.8814) (end 149.43836 117.78488) (width 0.254) (layer F.Cu) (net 5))
 (segment (start 126.57836 100.51288) (end 127.72136 101.65588) (width 0.254) (layer F.Cu) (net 5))
 (segment (start 127.72136 101.65588) (end 127.72136 104.17048) (width 0.254) (layer F.Cu) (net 5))
 (segment (start 126.57836 100.51288) (end 126.57836 96.7486) (width 0.254) (layer F.Cu) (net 5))
 (segment (start 137.3886 113.83772) (end 127.72136 104.17048) (width 0.254) (layer F.Cu) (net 5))
 (segment (start 145.4912 113.83772) (end 137.3886 113.83772) (width 0.254) (layer F.Cu) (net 5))
 (segment (start 149.43836 117.78488) (end 145.4912 113.83772) (width 0.254) (layer F.Cu) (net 5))
 (segment (start 157.05836 117.8814) (end 156.591 117.8814) (width 0.254) (layer F.Cu) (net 8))
 (segment (start 134.19836 99.9744) (end 135.48868 101.26472) (width 0.254) (layer F.Cu) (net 8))
 (segment (start 135.48868 101.26472) (end 135.48868 104.17048) (width 0.254) (layer F.Cu) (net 8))
 (segment (start 134.19836 99.9744) (end 134.19836 96.7486) (width 0.254) (layer F.Cu) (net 8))
 (segment (start 142.7226 111.4044) (end 135.48868 104.17048) (width 0.254) (layer F.Cu) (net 8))
 (segment (start 150.114 111.4044) (end 142.7226 111.4044) (width 0.254) (layer F.Cu) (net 8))
 (segment (start 156.591 117.8814) (end 150.114 111.4044) (width 0.254) (layer F.Cu) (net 8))
 (segment (start 113.87836 96.7486) (end 113.87836 100.66528) (width 0.254) (layer F.Cu) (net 1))
 (segment (start 141.9352 115.45824) (end 144.35836 117.8814) (width 0.254) (layer F.Cu) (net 1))
 (segment (start 126.65964 115.45824) (end 141.9352 115.45824) (width 0.254) (layer F.Cu) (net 1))
 (segment (start 115.14836 103.94696) (end 126.65964 115.45824) (width 0.254) (layer F.Cu) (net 1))
 (segment (start 115.14836 101.93528) (end 115.14836 103.94696) (width 0.254) (layer F.Cu) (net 1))
 (segment (start 113.87836 100.66528) (end 115.14836 101.93528) (width 0.254) (layer F.Cu) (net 1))
 (segment (start 116.41836 96.7486) (end 116.41836 97.42424) (width 0.254) (layer B.Cu) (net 2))
 (segment (start 112.07496 116.078) (end 113.87836 117.8814) (width 0.254) (layer B.Cu) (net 2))
 (segment (start 112.07496 101.76764) (end 112.07496 116.078) (width 0.254) (layer B.Cu) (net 2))
 (segment (start 116.41836 97.42424) (end 112.07496 101.76764) (width 0.254) (layer B.Cu) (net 2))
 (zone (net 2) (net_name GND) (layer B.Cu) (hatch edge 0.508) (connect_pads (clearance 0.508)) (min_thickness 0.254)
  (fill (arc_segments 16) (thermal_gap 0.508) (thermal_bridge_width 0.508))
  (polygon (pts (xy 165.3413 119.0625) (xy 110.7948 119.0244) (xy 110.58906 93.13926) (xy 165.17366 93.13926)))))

